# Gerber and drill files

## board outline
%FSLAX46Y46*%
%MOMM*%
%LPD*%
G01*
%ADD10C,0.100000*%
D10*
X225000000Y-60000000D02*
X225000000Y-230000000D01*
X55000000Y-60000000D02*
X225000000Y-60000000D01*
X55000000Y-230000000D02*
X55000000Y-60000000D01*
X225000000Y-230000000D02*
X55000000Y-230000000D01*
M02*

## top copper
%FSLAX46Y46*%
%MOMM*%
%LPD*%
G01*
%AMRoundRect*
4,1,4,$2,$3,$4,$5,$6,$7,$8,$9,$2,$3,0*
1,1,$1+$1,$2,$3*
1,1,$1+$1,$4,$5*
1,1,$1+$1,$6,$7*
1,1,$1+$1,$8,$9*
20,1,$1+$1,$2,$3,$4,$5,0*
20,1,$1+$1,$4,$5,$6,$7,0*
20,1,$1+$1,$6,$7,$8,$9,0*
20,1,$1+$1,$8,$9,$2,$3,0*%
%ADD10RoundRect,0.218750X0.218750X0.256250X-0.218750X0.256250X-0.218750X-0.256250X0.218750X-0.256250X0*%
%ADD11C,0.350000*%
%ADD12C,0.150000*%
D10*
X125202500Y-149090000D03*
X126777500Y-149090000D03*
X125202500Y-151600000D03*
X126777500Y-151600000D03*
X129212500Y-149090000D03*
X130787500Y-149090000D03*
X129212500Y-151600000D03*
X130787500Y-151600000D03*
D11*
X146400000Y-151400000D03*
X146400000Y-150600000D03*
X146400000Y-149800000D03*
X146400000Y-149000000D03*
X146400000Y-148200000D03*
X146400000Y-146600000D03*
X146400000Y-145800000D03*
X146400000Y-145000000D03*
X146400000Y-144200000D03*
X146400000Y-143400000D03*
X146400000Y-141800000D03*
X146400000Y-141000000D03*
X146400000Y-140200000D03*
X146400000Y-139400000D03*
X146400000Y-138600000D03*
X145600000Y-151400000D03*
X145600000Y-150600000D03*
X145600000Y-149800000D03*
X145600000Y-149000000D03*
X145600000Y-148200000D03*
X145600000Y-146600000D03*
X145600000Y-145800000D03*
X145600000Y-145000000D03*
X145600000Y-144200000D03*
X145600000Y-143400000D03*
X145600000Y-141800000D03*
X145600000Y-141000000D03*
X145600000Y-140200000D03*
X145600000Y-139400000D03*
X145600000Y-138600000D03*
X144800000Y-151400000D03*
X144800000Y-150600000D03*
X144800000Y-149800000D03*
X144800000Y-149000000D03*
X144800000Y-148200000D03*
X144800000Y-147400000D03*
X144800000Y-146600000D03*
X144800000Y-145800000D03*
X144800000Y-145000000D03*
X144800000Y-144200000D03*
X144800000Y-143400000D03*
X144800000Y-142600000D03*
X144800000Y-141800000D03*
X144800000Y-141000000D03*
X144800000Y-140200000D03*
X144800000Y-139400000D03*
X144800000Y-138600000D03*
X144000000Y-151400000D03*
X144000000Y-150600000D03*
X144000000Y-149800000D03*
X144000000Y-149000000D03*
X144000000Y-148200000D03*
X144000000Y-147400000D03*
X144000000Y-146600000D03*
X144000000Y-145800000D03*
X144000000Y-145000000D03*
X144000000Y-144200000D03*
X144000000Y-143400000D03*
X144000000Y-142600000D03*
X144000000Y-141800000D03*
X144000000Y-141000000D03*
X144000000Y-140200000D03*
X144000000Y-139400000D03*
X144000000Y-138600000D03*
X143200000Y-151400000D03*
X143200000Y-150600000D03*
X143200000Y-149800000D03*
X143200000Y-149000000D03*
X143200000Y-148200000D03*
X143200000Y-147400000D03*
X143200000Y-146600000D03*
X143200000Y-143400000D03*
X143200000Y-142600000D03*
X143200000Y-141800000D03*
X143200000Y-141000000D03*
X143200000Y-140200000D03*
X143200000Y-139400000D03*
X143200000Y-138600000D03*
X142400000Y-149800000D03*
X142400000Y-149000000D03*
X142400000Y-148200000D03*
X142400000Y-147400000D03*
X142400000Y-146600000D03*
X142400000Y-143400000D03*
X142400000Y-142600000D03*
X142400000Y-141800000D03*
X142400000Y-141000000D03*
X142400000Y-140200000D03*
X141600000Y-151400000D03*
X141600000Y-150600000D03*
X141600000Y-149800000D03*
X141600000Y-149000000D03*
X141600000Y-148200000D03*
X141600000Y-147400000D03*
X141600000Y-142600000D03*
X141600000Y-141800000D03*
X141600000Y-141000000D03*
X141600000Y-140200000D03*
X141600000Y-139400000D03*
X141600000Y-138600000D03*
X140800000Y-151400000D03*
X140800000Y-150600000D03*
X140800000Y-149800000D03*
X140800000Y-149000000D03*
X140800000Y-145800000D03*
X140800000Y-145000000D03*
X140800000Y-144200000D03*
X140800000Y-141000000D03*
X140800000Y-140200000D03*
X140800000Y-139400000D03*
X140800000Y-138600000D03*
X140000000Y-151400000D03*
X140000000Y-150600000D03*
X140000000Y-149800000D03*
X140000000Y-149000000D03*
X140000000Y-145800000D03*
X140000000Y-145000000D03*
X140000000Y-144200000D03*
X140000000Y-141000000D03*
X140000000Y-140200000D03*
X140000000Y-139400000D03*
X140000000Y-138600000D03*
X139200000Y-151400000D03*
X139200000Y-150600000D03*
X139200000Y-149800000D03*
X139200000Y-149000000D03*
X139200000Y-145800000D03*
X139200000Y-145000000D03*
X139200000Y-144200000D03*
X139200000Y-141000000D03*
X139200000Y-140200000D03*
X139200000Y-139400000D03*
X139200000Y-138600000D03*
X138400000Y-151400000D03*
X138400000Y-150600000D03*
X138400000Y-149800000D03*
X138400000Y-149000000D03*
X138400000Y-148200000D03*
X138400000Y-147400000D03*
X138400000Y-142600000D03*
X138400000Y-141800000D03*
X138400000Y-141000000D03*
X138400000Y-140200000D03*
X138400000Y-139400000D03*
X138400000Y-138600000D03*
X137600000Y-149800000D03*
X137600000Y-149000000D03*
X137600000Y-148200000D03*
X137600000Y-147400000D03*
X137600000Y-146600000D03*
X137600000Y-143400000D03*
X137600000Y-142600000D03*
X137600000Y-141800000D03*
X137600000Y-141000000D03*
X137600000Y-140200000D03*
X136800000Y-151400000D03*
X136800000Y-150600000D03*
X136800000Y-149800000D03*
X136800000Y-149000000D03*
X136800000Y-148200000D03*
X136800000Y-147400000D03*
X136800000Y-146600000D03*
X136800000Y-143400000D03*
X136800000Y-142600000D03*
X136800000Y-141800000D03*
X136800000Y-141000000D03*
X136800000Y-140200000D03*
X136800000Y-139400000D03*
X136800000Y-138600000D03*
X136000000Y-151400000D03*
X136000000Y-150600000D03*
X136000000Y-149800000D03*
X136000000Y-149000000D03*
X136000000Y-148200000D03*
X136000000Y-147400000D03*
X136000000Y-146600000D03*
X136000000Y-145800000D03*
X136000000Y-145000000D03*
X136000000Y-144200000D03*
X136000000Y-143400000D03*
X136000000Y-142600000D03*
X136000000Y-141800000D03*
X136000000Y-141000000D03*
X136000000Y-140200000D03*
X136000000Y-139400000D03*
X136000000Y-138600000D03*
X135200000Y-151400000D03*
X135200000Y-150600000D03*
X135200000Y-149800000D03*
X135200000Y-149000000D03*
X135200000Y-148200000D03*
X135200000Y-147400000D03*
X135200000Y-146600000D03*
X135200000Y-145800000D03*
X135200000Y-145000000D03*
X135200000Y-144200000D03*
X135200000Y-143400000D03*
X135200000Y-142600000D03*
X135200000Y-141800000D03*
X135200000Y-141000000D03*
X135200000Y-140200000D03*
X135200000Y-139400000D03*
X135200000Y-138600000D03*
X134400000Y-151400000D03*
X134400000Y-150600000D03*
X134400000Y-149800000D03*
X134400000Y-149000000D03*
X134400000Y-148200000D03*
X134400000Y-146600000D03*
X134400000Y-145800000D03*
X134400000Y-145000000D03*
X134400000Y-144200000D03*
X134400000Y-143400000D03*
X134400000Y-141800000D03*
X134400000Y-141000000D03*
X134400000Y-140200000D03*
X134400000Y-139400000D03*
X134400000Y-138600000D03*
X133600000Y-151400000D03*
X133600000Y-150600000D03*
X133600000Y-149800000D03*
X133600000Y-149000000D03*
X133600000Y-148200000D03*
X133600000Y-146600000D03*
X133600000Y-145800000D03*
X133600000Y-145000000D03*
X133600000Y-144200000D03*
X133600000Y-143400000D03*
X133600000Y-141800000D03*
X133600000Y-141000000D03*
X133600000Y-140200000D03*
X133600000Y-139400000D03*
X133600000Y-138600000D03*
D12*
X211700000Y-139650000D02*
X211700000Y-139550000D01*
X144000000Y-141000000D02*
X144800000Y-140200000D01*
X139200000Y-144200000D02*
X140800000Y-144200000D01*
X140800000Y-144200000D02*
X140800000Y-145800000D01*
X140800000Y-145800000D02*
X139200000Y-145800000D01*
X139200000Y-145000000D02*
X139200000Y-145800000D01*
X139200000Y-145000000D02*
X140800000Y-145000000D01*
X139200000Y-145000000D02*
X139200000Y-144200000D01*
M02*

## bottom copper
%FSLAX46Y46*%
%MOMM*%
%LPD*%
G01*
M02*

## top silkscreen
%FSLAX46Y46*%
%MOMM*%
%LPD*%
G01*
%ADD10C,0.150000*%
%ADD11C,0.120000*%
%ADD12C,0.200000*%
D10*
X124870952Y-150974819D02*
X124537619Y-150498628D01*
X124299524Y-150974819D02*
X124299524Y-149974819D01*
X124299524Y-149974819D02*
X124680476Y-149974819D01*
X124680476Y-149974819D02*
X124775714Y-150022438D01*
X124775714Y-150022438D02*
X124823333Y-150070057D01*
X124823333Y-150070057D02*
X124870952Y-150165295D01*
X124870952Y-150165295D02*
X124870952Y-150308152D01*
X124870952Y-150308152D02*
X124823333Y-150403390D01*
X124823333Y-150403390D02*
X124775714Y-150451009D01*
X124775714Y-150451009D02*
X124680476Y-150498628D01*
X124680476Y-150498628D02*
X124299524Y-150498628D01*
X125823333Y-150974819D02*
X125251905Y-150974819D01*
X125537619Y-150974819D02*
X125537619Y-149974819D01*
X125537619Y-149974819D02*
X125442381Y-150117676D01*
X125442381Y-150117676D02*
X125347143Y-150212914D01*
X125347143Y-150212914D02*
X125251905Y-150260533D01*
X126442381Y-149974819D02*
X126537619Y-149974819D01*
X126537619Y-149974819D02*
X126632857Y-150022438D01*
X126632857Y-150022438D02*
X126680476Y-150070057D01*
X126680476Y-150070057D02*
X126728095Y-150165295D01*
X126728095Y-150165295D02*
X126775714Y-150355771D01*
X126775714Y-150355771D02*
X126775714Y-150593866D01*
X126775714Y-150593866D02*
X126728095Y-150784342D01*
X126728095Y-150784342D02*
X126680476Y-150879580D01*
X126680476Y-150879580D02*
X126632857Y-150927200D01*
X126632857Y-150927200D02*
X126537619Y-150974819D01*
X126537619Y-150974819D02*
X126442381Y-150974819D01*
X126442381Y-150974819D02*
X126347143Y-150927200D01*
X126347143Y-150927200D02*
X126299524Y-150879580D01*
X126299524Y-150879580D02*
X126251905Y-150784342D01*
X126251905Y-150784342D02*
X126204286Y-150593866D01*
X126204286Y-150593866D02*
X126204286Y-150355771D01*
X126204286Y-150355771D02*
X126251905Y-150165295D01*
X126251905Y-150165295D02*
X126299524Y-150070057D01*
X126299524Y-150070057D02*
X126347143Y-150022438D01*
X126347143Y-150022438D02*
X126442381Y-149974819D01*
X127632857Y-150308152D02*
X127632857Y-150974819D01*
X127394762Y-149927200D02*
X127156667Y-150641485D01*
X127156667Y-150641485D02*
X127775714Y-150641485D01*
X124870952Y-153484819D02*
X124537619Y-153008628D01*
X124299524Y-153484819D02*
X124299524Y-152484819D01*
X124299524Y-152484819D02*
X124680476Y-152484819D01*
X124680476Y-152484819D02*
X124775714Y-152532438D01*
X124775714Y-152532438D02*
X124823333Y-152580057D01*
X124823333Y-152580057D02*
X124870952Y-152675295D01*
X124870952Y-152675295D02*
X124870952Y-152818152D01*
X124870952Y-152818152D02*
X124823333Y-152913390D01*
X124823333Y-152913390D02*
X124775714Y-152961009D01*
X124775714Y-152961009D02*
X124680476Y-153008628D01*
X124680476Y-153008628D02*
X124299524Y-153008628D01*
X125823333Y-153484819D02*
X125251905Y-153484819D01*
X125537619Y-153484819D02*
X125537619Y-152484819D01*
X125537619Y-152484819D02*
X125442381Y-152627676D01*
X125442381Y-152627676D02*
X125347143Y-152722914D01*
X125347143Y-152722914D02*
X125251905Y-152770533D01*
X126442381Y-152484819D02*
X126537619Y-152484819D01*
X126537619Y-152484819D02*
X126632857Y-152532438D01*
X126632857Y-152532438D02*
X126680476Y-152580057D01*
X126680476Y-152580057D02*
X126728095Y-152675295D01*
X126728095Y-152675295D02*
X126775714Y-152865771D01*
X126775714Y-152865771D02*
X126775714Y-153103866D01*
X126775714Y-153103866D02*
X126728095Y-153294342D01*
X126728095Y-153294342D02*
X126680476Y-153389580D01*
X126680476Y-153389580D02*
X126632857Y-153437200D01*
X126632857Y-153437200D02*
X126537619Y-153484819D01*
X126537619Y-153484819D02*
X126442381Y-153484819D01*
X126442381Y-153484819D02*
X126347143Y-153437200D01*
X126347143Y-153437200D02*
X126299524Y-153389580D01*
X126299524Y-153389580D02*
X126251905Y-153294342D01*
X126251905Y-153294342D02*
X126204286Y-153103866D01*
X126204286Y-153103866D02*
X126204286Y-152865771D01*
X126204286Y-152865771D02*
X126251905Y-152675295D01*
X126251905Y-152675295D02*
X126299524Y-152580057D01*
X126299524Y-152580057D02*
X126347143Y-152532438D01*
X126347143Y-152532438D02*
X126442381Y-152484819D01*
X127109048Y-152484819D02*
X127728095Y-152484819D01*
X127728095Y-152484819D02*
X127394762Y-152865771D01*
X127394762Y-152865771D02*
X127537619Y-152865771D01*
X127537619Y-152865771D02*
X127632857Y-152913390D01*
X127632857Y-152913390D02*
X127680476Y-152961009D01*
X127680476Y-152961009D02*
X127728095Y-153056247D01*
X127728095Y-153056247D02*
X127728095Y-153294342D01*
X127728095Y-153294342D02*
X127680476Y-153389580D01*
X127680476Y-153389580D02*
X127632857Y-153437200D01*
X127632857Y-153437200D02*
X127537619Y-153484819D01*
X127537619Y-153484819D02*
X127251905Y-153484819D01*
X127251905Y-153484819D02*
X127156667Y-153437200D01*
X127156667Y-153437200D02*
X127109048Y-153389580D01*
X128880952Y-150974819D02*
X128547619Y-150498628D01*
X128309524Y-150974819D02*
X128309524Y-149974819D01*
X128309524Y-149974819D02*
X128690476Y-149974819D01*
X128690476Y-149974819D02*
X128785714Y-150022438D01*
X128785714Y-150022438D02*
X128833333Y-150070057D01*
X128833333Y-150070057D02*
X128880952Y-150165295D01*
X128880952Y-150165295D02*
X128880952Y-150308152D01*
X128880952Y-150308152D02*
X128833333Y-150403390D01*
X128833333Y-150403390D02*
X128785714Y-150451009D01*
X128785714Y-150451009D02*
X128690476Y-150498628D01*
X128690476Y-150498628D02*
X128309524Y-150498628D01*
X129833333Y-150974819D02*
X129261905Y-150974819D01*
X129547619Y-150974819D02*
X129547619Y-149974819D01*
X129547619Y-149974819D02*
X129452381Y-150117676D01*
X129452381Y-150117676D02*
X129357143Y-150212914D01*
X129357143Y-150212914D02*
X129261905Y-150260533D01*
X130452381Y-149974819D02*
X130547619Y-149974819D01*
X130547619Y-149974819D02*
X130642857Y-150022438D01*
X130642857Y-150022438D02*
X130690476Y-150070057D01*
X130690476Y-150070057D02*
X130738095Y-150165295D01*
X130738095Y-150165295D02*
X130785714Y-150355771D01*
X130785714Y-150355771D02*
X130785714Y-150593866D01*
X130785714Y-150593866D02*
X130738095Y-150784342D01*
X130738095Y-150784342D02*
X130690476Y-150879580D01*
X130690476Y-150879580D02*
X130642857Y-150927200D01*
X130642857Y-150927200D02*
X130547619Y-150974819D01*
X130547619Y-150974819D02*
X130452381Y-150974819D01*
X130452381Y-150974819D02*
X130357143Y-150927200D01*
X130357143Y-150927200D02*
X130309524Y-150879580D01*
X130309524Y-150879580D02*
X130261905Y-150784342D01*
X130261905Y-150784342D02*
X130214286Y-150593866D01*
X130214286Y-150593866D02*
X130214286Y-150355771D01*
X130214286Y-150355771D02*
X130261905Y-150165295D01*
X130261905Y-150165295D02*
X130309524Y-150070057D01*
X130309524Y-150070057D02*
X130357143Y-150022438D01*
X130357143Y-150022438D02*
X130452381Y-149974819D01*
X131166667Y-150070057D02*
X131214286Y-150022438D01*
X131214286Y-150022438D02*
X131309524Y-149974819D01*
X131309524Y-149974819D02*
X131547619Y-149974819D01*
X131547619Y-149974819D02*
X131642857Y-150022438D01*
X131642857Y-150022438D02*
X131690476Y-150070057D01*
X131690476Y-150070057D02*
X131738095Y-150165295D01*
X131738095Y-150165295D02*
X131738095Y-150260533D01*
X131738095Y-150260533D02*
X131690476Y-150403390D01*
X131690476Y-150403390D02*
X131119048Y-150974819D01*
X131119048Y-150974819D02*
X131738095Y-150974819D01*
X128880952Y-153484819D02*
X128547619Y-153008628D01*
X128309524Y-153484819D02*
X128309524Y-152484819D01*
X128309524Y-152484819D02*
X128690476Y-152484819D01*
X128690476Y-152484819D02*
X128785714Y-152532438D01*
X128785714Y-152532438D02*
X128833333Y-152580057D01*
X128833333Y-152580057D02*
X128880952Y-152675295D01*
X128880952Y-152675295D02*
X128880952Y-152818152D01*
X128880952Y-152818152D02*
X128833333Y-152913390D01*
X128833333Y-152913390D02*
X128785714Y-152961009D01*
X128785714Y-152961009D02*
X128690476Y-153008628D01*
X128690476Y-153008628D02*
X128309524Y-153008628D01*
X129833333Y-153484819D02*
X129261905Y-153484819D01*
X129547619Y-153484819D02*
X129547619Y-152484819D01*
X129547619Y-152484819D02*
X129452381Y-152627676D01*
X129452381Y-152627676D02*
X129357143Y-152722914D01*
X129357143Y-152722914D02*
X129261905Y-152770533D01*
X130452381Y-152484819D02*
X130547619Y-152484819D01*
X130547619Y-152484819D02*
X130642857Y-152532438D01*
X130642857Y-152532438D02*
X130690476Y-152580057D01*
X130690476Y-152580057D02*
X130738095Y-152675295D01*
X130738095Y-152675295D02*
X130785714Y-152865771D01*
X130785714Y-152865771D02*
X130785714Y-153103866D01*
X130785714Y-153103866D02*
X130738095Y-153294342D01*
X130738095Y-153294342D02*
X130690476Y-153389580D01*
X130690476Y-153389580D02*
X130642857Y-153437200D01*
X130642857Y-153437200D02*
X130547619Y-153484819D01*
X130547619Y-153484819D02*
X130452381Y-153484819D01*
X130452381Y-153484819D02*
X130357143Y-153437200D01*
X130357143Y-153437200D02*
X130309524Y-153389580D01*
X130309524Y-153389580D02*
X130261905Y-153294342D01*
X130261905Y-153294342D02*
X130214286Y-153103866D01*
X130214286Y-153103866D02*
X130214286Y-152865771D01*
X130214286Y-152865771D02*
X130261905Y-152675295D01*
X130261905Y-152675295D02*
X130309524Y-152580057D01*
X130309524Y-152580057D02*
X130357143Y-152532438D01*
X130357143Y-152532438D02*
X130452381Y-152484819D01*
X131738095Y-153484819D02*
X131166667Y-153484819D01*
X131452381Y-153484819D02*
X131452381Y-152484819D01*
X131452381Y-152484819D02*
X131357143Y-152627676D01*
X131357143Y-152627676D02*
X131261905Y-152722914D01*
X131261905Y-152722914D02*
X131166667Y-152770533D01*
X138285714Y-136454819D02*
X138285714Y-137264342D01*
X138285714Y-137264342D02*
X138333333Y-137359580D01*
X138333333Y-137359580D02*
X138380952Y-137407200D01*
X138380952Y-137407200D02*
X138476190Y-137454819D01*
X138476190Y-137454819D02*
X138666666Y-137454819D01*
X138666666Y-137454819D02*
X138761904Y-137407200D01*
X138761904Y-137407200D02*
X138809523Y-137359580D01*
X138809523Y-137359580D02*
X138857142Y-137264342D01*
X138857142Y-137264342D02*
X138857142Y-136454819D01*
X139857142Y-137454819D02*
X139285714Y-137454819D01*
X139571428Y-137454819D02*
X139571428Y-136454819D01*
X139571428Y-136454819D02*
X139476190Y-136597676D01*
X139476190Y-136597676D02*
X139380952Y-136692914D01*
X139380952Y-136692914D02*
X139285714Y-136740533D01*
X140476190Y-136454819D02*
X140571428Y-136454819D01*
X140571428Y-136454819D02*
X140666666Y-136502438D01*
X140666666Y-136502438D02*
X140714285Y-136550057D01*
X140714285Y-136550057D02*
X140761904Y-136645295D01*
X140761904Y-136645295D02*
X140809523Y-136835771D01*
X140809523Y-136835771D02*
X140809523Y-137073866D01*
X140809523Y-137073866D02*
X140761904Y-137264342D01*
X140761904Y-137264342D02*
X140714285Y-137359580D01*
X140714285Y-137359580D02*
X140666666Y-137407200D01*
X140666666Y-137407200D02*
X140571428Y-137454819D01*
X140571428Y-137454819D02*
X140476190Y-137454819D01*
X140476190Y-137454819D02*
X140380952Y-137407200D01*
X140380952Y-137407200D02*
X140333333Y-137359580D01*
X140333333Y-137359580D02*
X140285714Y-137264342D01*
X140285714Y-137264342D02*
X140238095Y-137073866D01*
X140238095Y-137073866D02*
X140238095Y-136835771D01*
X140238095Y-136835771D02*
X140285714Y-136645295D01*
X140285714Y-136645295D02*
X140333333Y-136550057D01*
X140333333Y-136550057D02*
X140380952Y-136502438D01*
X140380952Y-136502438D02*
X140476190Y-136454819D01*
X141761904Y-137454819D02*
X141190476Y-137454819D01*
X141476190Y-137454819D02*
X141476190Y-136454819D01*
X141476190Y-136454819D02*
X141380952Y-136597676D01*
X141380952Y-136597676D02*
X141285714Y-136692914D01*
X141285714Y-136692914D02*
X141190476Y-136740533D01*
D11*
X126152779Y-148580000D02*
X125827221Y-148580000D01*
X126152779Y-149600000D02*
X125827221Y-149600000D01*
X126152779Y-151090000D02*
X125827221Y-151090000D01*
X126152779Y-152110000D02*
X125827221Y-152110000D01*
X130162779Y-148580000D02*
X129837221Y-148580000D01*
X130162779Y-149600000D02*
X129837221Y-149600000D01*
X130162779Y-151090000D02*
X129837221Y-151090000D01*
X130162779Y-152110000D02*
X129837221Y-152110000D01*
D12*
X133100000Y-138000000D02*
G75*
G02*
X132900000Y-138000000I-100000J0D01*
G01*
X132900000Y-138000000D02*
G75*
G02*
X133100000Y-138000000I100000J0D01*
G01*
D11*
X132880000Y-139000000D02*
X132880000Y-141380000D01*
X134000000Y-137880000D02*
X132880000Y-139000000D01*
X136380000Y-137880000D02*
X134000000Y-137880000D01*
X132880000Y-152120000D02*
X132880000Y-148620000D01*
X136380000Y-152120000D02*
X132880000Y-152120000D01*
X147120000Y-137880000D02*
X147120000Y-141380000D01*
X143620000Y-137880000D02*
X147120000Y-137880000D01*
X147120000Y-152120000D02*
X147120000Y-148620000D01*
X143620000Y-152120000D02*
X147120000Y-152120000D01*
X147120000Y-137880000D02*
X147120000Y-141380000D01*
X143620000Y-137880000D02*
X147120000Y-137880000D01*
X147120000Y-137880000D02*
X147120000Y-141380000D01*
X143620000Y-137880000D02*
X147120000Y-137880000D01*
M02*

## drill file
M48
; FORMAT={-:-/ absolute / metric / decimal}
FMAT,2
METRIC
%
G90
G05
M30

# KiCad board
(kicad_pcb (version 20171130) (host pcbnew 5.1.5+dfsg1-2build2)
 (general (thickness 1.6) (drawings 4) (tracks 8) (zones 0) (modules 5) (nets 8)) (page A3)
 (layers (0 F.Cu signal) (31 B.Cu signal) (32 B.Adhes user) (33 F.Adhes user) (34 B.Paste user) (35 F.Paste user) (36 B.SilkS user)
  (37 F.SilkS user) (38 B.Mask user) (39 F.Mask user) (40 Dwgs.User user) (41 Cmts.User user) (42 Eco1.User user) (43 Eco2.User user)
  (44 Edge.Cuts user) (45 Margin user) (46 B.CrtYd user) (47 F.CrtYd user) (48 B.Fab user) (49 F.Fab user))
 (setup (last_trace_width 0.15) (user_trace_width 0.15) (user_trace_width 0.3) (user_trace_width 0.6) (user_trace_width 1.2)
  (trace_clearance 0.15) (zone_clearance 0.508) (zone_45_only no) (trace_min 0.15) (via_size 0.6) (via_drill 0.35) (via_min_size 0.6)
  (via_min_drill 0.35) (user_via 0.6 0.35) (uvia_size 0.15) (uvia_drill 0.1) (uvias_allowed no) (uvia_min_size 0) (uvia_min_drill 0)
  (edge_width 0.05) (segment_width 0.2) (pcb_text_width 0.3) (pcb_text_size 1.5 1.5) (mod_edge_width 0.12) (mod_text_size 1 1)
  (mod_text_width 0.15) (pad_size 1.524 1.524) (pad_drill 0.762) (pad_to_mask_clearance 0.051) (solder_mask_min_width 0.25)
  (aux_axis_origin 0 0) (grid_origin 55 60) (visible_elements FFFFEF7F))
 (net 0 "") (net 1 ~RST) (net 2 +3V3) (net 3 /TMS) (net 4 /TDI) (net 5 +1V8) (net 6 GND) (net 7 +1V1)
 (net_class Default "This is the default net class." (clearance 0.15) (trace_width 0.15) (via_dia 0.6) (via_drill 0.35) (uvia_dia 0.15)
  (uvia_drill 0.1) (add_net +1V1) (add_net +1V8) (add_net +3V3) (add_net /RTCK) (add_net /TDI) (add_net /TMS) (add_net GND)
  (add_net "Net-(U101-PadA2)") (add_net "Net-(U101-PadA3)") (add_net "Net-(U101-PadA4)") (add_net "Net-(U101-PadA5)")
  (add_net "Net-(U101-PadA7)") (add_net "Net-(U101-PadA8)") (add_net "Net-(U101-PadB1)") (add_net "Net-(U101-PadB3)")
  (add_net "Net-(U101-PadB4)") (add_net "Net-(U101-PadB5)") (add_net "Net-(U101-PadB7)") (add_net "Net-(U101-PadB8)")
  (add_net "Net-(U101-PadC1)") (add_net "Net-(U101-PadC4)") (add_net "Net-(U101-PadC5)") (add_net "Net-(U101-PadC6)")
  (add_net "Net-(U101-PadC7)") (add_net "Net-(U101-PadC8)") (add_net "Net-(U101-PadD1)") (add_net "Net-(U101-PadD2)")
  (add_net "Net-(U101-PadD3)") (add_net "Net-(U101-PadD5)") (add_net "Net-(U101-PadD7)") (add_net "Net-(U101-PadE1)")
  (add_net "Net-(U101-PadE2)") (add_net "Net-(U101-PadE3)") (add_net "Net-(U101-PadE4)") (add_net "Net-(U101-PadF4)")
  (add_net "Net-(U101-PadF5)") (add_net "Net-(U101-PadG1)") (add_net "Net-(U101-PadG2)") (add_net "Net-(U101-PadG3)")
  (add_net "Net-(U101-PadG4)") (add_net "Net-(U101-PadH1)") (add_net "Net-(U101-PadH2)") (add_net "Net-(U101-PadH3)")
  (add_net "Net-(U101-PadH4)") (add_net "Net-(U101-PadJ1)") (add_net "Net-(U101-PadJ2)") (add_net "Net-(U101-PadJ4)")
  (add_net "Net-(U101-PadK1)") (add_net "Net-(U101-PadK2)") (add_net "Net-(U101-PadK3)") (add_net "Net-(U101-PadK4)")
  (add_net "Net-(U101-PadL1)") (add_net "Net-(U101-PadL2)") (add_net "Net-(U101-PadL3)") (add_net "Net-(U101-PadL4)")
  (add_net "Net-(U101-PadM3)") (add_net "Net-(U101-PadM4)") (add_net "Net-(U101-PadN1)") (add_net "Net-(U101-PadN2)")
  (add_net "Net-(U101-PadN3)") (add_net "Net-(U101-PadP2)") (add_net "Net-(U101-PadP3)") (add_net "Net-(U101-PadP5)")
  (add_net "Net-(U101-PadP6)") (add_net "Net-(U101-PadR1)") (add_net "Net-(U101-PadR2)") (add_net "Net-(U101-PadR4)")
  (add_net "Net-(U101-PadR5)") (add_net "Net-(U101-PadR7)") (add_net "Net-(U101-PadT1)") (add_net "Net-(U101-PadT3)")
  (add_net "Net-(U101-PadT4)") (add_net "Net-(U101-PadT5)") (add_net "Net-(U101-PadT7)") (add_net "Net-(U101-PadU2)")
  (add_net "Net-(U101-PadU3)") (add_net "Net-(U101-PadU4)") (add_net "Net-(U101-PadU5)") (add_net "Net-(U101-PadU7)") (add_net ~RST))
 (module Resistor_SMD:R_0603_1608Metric (layer F.Cu) (at 125.99 149.09 180)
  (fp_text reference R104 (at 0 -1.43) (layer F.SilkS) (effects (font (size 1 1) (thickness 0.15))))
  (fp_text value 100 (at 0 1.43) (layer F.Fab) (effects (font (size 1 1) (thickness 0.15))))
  (fp_line (start -0.162779 0.51) (end 0.162779 0.51) (layer F.SilkS) (width 0.12))
  (fp_line (start -0.162779 -0.51) (end 0.162779 -0.51) (layer F.SilkS) (width 0.12))
  (pad 2 smd roundrect (at 0.7875 0 180) (size 0.875 0.95) (layers F.Cu F.Paste F.Mask) (roundrect_rratio 0.25))
  (pad 1 smd roundrect (at -0.7875 0 180) (size 0.875 0.95) (layers F.Cu F.Paste F.Mask) (roundrect_rratio 0.25) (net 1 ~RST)))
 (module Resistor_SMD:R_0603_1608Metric (layer F.Cu) (at 125.99 151.6 180)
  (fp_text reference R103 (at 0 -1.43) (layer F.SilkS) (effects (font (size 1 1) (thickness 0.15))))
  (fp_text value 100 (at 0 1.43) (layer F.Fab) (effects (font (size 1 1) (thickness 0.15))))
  (fp_line (start -0.162779 0.51) (end 0.162779 0.51) (layer F.SilkS) (width 0.12))
  (fp_line (start -0.162779 -0.51) (end 0.162779 -0.51) (layer F.SilkS) (width 0.12))
  (pad 2 smd roundrect (at 0.7875 0 180) (size 0.875 0.95) (layers F.Cu F.Paste F.Mask) (roundrect_rratio 0.25) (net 1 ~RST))
  (pad 1 smd roundrect (at -0.7875 0 180) (size 0.875 0.95) (layers F.Cu F.Paste F.Mask) (roundrect_rratio 0.25) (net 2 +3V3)))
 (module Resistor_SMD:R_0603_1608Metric (layer F.Cu) (at 130 149.09 180)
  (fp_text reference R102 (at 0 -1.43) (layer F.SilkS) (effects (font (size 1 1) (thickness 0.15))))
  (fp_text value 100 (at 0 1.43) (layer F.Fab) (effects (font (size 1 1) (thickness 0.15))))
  (fp_line (start -0.162779 0.51) (end 0.162779 0.51) (layer F.SilkS) (width 0.12))
  (fp_line (start -0.162779 -0.51) (end 0.162779 -0.51) (layer F.SilkS) (width 0.12))
  (pad 2 smd roundrect (at 0.7875 0 180) (size 0.875 0.95) (layers F.Cu F.Paste F.Mask) (roundrect_rratio 0.25) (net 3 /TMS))
  (pad 1 smd roundrect (at -0.7875 0 180) (size 0.875 0.95) (layers F.Cu F.Paste F.Mask) (roundrect_rratio 0.25) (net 2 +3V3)))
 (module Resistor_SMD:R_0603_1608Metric (layer F.Cu) (at 130 151.6 180)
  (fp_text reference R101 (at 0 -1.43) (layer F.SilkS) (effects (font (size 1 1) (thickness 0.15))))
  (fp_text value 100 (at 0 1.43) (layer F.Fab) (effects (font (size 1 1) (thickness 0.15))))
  (fp_line (start -0.162779 0.51) (end 0.162779 0.51) (layer F.SilkS) (width 0.12))
  (fp_line (start -0.162779 -0.51) (end 0.162779 -0.51) (layer F.SilkS) (width 0.12))
  (pad 2 smd roundrect (at 0.7875 0 180) (size 0.875 0.95) (layers F.Cu F.Paste F.Mask) (roundrect_rratio 0.25) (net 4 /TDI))
  (pad 1 smd roundrect (at -0.7875 0 180) (size 0.875 0.95) (layers F.Cu F.Paste F.Mask) (roundrect_rratio 0.25) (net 2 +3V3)))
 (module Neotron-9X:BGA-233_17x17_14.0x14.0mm (layer F.Cu) (at 140 145)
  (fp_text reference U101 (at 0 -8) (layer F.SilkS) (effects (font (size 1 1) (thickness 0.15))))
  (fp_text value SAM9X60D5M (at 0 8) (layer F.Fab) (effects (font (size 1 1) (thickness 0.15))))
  (fp_circle (center -7 -7) (end -7 -6.9) (layer F.SilkS) (width 0.2))
  (fp_line (start -7.12 -6) (end -7.12 -3.62) (layer F.SilkS) (width 0.12))
  (fp_line (start -6 -7.12) (end -7.12 -6) (layer F.SilkS) (width 0.12))
  (fp_line (start -3.62 -7.12) (end -6 -7.12) (layer F.SilkS) (width 0.12))
  (fp_line (start -7.12 7.12) (end -7.12 3.62) (layer F.SilkS) (width 0.12))
  (fp_line (start -3.62 7.12) (end -7.12 7.12) (layer F.SilkS) (width 0.12))
  (fp_line (start 7.12 -7.12) (end 7.12 -3.62) (layer F.SilkS) (width 0.12))
  (fp_line (start 3.62 -7.12) (end 7.12 -7.12) (layer F.SilkS) (width 0.12))
  (fp_line (start 7.12 7.12) (end 7.12 3.62) (layer F.SilkS) (width 0.12))
  (fp_line (start 3.62 7.12) (end 7.12 7.12) (layer F.SilkS) (width 0.12))
  (fp_line (start 7.12 -7.12) (end 7.12 -3.62) (layer F.SilkS) (width 0.12))
  (fp_line (start 3.62 -7.12) (end 7.12 -7.12) (layer F.SilkS) (width 0.12))
  (fp_line (start 7.12 -7.12) (end 7.12 -3.62) (layer F.SilkS) (width 0.12))
  (fp_line (start 3.62 -7.12) (end 7.12 -7.12) (layer F.SilkS) (width 0.12))
  (pad U17 smd circle (at 6.4 6.4) (size 0.35 0.35) (layers F.Cu F.Paste F.Mask))
  (pad T17 smd circle (at 6.4 5.6) (size 0.35 0.35) (layers F.Cu F.Paste F.Mask))
  (pad R17 smd circle (at 6.4 4.8) (size 0.35 0.35) (layers F.Cu F.Paste F.Mask))
  (pad P17 smd circle (at 6.4 4) (size 0.35 0.35) (layers F.Cu F.Paste F.Mask))
  (pad N17 smd circle (at 6.4 3.2) (size 0.35 0.35) (layers F.Cu F.Paste F.Mask))
  (pad L17 smd circle (at 6.4 1.6) (size 0.35 0.35) (layers F.Cu F.Paste F.Mask))
  (pad K17 smd circle (at 6.4 0.8) (size 0.35 0.35) (layers F.Cu F.Paste F.Mask))
  (pad J17 smd circle (at 6.4 0) (size 0.35 0.35) (layers F.Cu F.Paste F.Mask))
  (pad H17 smd circle (at 6.4 -0.8) (size 0.35 0.35) (layers F.Cu F.Paste F.Mask))
  (pad G17 smd circle (at 6.4 -1.6) (size 0.35 0.35) (layers F.Cu F.Paste F.Mask))
  (pad E17 smd circle (at 6.4 -3.2) (size 0.35 0.35) (layers F.Cu F.Paste F.Mask))
  (pad D17 smd circle (at 6.4 -4) (size 0.35 0.35) (layers F.Cu F.Paste F.Mask))
  (pad C17 smd circle (at 6.4 -4.8) (size 0.35 0.35) (layers F.Cu F.Paste F.Mask))
  (pad B17 smd circle (at 6.4 -5.6) (size 0.35 0.35) (layers F.Cu F.Paste F.Mask) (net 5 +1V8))
  (pad A17 smd circle (at 6.4 -6.4) (size 0.35 0.35) (layers F.Cu F.Paste F.Mask) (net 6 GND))
  (pad U16 smd circle (at 5.6 6.4) (size 0.35 0.35) (layers F.Cu F.Paste F.Mask))
  (pad T16 smd circle (at 5.6 5.6) (size 0.35 0.35) (layers F.Cu F.Paste F.Mask) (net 6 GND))
  (pad R16 smd circle (at 5.6 4.8) (size 0.35 0.35) (layers F.Cu F.Paste F.Mask) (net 6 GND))
  (pad P16 smd circle (at 5.6 4) (size 0.35 0.35) (layers F.Cu F.Paste F.Mask))
  (pad N16 smd circle (at 5.6 3.2) (size 0.35 0.35) (layers F.Cu F.Paste F.Mask) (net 3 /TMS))
  (pad L16 smd circle (at 5.6 1.6) (size 0.35 0.35) (layers F.Cu F.Paste F.Mask))
  (pad K16 smd circle (at 5.6 0.8) (size 0.35 0.35) (layers F.Cu F.Paste F.Mask))
  (pad J16 smd circle (at 5.6 0) (size 0.35 0.35) (layers F.Cu F.Paste F.Mask))
  (pad H16 smd circle (at 5.6 -0.8) (size 0.35 0.35) (layers F.Cu F.Paste F.Mask))
  (pad G16 smd circle (at 5.6 -1.6) (size 0.35 0.35) (layers F.Cu F.Paste F.Mask))
  (pad E16 smd circle (at 5.6 -3.2) (size 0.35 0.35) (layers F.Cu F.Paste F.Mask))
  (pad D16 smd circle (at 5.6 -4) (size 0.35 0.35) (layers F.Cu F.Paste F.Mask))
  (pad C16 smd circle (at 5.6 -4.8) (size 0.35 0.35) (layers F.Cu F.Paste F.Mask) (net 5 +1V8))
  (pad B16 smd circle (at 5.6 -5.6) (size 0.35 0.35) (layers F.Cu F.Paste F.Mask) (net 6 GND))
  (pad A16 smd circle (at 5.6 -6.4) (size 0.35 0.35) (layers F.Cu F.Paste F.Mask) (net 5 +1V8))
  (pad U15 smd circle (at 4.8 6.4) (size 0.35 0.35) (layers F.Cu F.Paste F.Mask) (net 6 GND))
  (pad T15 smd circle (at 4.8 5.6) (size 0.35 0.35) (layers F.Cu F.Paste F.Mask))
  (pad R15 smd circle (at 4.8 4.8) (size 0.35 0.35) (layers F.Cu F.Paste F.Mask) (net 6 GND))
  (pad P15 smd circle (at 4.8 4) (size 0.35 0.35) (layers F.Cu F.Paste F.Mask))
  (pad N15 smd circle (at 4.8 3.2) (size 0.35 0.35) (layers F.Cu F.Paste F.Mask))
  (pad M15 smd circle (at 4.8 2.4) (size 0.35 0.35) (layers F.Cu F.Paste F.Mask))
  (pad L15 smd circle (at 4.8 1.6) (size 0.35 0.35) (layers F.Cu F.Paste F.Mask) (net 4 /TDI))
  (pad K15 smd circle (at 4.8 0.8) (size 0.35 0.35) (layers F.Cu F.Paste F.Mask))
  (pad J15 smd circle (at 4.8 0) (size 0.35 0.35) (layers F.Cu F.Paste F.Mask) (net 6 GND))
  (pad H15 smd circle (at 4.8 -0.8) (size 0.35 0.35) (layers F.Cu F.Paste F.Mask))
  (pad G15 smd circle (at 4.8 -1.6) (size 0.35 0.35) (layers F.Cu F.Paste F.Mask))
  (pad F15 smd circle (at 4.8 -2.4) (size 0.35 0.35) (layers F.Cu F.Paste F.Mask) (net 6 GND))
  (pad E15 smd circle (at 4.8 -3.2) (size 0.35 0.35) (layers F.Cu F.Paste F.Mask))
  (pad D15 smd circle (at 4.8 -4) (size 0.35 0.35) (layers F.Cu F.Paste F.Mask) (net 5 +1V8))
  (pad C15 smd circle (at 4.8 -4.8) (size 0.35 0.35) (layers F.Cu F.Paste F.Mask) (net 6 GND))
  (pad B15 smd circle (at 4.8 -5.6) (size 0.35 0.35) (layers F.Cu F.Paste F.Mask) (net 5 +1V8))
  (pad A15 smd circle (at 4.8 -6.4) (size 0.35 0.35) (layers F.Cu F.Paste F.Mask) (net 6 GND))
  (pad U14 smd circle (at 4 6.4) (size 0.35 0.35) (layers F.Cu F.Paste F.Mask))
  (pad T14 smd circle (at 4 5.6) (size 0.35 0.35) (layers F.Cu F.Paste F.Mask))
  (pad R14 smd circle (at 4 4.8) (size 0.35 0.35) (layers F.Cu F.Paste F.Mask))
  (pad P14 smd circle (at 4 4) (size 0.35 0.35) (layers F.Cu F.Paste F.Mask) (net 6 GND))
  (pad N14 smd circle (at 4 3.2) (size 0.35 0.35) (layers F.Cu F.Paste F.Mask))
  (pad M14 smd circle (at 4 2.4) (size 0.35 0.35) (layers F.Cu F.Paste F.Mask) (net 6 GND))
  (pad L14 smd circle (at 4 1.6) (size 0.35 0.35) (layers F.Cu F.Paste F.Mask) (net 6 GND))
  (pad K14 smd circle (at 4 0.8) (size 0.35 0.35) (layers F.Cu F.Paste F.Mask))
  (pad J14 smd circle (at 4 0) (size 0.35 0.35) (layers F.Cu F.Paste F.Mask))
  (pad H14 smd circle (at 4 -0.8) (size 0.35 0.35) (layers F.Cu F.Paste F.Mask))
  (pad G14 smd circle (at 4 -1.6) (size 0.35 0.35) (layers F.Cu F.Paste F.Mask))
  (pad F14 smd circle (at 4 -2.4) (size 0.35 0.35) (layers F.Cu F.Paste F.Mask))
  (pad E14 smd circle (at 4 -3.2) (size 0.35 0.35) (layers F.Cu F.Paste F.Mask))
  (pad D14 smd circle (at 4 -4) (size 0.35 0.35) (layers F.Cu F.Paste F.Mask) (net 6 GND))
  (pad C14 smd circle (at 4 -4.8) (size 0.35 0.35) (layers F.Cu F.Paste F.Mask) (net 5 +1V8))
  (pad B14 smd circle (at 4 -5.6) (size 0.35 0.35) (layers F.Cu F.Paste F.Mask) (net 6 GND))
  (pad A14 smd circle (at 4 -6.4) (size 0.35 0.35) (layers F.Cu F.Paste F.Mask))
  (pad U13 smd circle (at 3.2 6.4) (size 0.35 0.35) (layers F.Cu F.Paste F.Mask))
  (pad T13 smd circle (at 3.2 5.6) (size 0.35 0.35) (layers F.Cu F.Paste F.Mask))
  (pad R13 smd circle (at 3.2 4.8) (size 0.35 0.35) (layers F.Cu F.Paste F.Mask))
  (pad P13 smd circle (at 3.2 4) (size 0.35 0.35) (layers F.Cu F.Paste F.Mask))
  (pad N13 smd circle (at 3.2 3.2) (size 0.35 0.35) (layers F.Cu F.Paste F.Mask) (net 6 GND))
  (pad M13 smd circle (at 3.2 2.4) (size 0.35 0.35) (layers F.Cu F.Paste F.Mask) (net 6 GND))
  (pad L13 smd circle (at 3.2 1.6) (size 0.35 0.35) (layers F.Cu F.Paste F.Mask) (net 6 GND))
  (pad G13 smd circle (at 3.2 -1.6) (size 0.35 0.35) (layers F.Cu F.Paste F.Mask) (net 5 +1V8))
  (pad F13 smd circle (at 3.2 -2.4) (size 0.35 0.35) (layers F.Cu F.Paste F.Mask) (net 5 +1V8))
  (pad E13 smd circle (at 3.2 -3.2) (size 0.35 0.35) (layers F.Cu F.Paste F.Mask) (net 6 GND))
  (pad D13 smd circle (at 3.2 -4) (size 0.35 0.35) (layers F.Cu F.Paste F.Mask) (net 5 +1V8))
  (pad C13 smd circle (at 3.2 -4.8) (size 0.35 0.35) (layers F.Cu F.Paste F.Mask) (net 6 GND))
  (pad B13 smd circle (at 3.2 -5.6) (size 0.35 0.35) (layers F.Cu F.Paste F.Mask) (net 6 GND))
  (pad A13 smd circle (at 3.2 -6.4) (size 0.35 0.35) (layers F.Cu F.Paste F.Mask) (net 6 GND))
  (pad R12 smd circle (at 2.4 4.8) (size 0.35 0.35) (layers F.Cu F.Paste F.Mask))
  (pad P12 smd circle (at 2.4 4) (size 0.35 0.35) (layers F.Cu F.Paste F.Mask))
  (pad N12 smd circle (at 2.4 3.2) (size 0.35 0.35) (layers F.Cu F.Paste F.Mask) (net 6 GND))
  (pad M12 smd circle (at 2.4 2.4) (size 0.35 0.35) (layers F.Cu F.Paste F.Mask) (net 6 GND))
  (pad L12 smd circle (at 2.4 1.6) (size 0.35 0.35) (layers F.Cu F.Paste F.Mask) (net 6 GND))
  (pad G12 smd circle (at 2.4 -1.6) (size 0.35 0.35) (layers F.Cu F.Paste F.Mask) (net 6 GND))
  (pad F12 smd circle (at 2.4 -2.4) (size 0.35 0.35) (layers F.Cu F.Paste F.Mask) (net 6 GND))
  (pad E12 smd circle (at 2.4 -3.2) (size 0.35 0.35) (layers F.Cu F.Paste F.Mask) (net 5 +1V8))
  (pad D12 smd circle (at 2.4 -4) (size 0.35 0.35) (layers F.Cu F.Paste F.Mask))
  (pad C12 smd circle (at 2.4 -4.8) (size 0.35 0.35) (layers F.Cu F.Paste F.Mask) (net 6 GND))
  (pad U11 smd circle (at 1.6 6.4) (size 0.35 0.35) (layers F.Cu F.Paste F.Mask))
  (pad T11 smd circle (at 1.6 5.6) (size 0.35 0.35) (layers F.Cu F.Paste F.Mask))
  (pad R11 smd circle (at 1.6 4.8) (size 0.35 0.35) (layers F.Cu F.Paste F.Mask) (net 6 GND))
  (pad P11 smd circle (at 1.6 4) (size 0.35 0.35) (layers F.Cu F.Paste F.Mask))
  (pad N11 smd circle (at 1.6 3.2) (size 0.35 0.35) (layers F.Cu F.Paste F.Mask))
  (pad M11 smd circle (at 1.6 2.4) (size 0.35 0.35) (layers F.Cu F.Paste F.Mask) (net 6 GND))
  (pad F11 smd circle (at 1.6 -2.4) (size 0.35 0.35) (layers F.Cu F.Paste F.Mask) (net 6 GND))
  (pad E11 smd circle (at 1.6 -3.2) (size 0.35 0.35) (layers F.Cu F.Paste F.Mask) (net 5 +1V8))
  (pad D11 smd circle (at 1.6 -4) (size 0.35 0.35) (layers F.Cu F.Paste F.Mask))
  (pad C11 smd circle (at 1.6 -4.8) (size 0.35 0.35) (layers F.Cu F.Paste F.Mask))
  (pad B11 smd circle (at 1.6 -5.6) (size 0.35 0.35) (layers F.Cu F.Paste F.Mask))
  (pad A11 smd circle (at 1.6 -6.4) (size 0.35 0.35) (layers F.Cu F.Paste F.Mask))
  (pad U10 smd circle (at 0.8 6.4) (size 0.35 0.35) (layers F.Cu F.Paste F.Mask))
  (pad T10 smd circle (at 0.8 5.6) (size 0.35 0.35) (layers F.Cu F.Paste F.Mask))
  (pad R10 smd circle (at 0.8 4.8) (size 0.35 0.35) (layers F.Cu F.Paste F.Mask))
  (pad P10 smd circle (at 0.8 4) (size 0.35 0.35) (layers F.Cu F.Paste F.Mask) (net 6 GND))
  (pad K10 smd circle (at 0.8 0.8) (size 0.35 0.35) (layers F.Cu F.Paste F.Mask) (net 6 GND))
  (pad J10 smd circle (at 0.8 0) (size 0.35 0.35) (layers F.Cu F.Paste F.Mask) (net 6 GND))
  (pad H10 smd circle (at 0.8 -0.8) (size 0.35 0.35) (layers F.Cu F.Paste F.Mask) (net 6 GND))
  (pad D10 smd circle (at 0.8 -4) (size 0.35 0.35) (layers F.Cu F.Paste F.Mask))
  (pad C10 smd circle (at 0.8 -4.8) (size 0.35 0.35) (layers F.Cu F.Paste F.Mask))
  (pad B10 smd circle (at 0.8 -5.6) (size 0.35 0.35) (layers F.Cu F.Paste F.Mask))
  (pad A10 smd circle (at 0.8 -6.4) (size 0.35 0.35) (layers F.Cu F.Paste F.Mask))
  (pad U9 smd circle (at 0 6.4) (size 0.35 0.35) (layers F.Cu F.Paste F.Mask))
  (pad T9 smd circle (at 0 5.6) (size 0.35 0.35) (layers F.Cu F.Paste F.Mask))
  (pad R9 smd circle (at 0 4.8) (size 0.35 0.35) (layers F.Cu F.Paste F.Mask) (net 6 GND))
  (pad P9 smd circle (at 0 4) (size 0.35 0.35) (layers F.Cu F.Paste F.Mask))
  (pad K9 smd circle (at 0 0.8) (size 0.35 0.35) (layers F.Cu F.Paste F.Mask) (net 6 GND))
  (pad J9 smd circle (at 0 0) (size 0.35 0.35) (layers F.Cu F.Paste F.Mask) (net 6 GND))
  (pad H9 smd circle (at 0 -0.8) (size 0.35 0.35) (layers F.Cu F.Paste F.Mask) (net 6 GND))
  (pad D9 smd circle (at 0 -4) (size 0.35 0.35) (layers F.Cu F.Paste F.Mask))
  (pad C9 smd circle (at 0 -4.8) (size 0.35 0.35) (layers F.Cu F.Paste F.Mask) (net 6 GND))
  (pad B9 smd circle (at 0 -5.6) (size 0.35 0.35) (layers F.Cu F.Paste F.Mask))
  (pad A9 smd circle (at 0 -6.4) (size 0.35 0.35) (layers F.Cu F.Paste F.Mask))
  (pad U8 smd circle (at -0.8 6.4) (size 0.35 0.35) (layers F.Cu F.Paste F.Mask))
  (pad T8 smd circle (at -0.8 5.6) (size 0.35 0.35) (layers F.Cu F.Paste F.Mask))
  (pad R8 smd circle (at -0.8 4.8) (size 0.35 0.35) (layers F.Cu F.Paste F.Mask))
  (pad P8 smd circle (at -0.8 4) (size 0.35 0.35) (layers F.Cu F.Paste F.Mask))
  (pad K8 smd circle (at -0.8 0.8) (size 0.35 0.35) (layers F.Cu F.Paste F.Mask) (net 6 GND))
  (pad J8 smd circle (at -0.8 0) (size 0.35 0.35) (layers F.Cu F.Paste F.Mask) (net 6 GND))
  (pad H8 smd circle (at -0.8 -0.8) (size 0.35 0.35) (layers F.Cu F.Paste F.Mask) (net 6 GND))
  (pad D8 smd circle (at -0.8 -4) (size 0.35 0.35) (layers F.Cu F.Paste F.Mask) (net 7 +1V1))
  (pad C8 smd circle (at -0.8 -4.8) (size 0.35 0.35) (layers F.Cu F.Paste F.Mask))
  (pad B8 smd circle (at -0.8 -5.6) (size 0.35 0.35) (layers F.Cu F.Paste F.Mask))
  (pad A8 smd circle (at -0.8 -6.4) (size 0.35 0.35) (layers F.Cu F.Paste F.Mask))
  (pad U7 smd circle (at -1.6 6.4) (size 0.35 0.35) (layers F.Cu F.Paste F.Mask))
  (pad T7 smd circle (at -1.6 5.6) (size 0.35 0.35) (layers F.Cu F.Paste F.Mask))
  (pad R7 smd circle (at -1.6 4.8) (size 0.35 0.35) (layers F.Cu F.Paste F.Mask))
  (pad P7 smd circle (at -1.6 4) (size 0.35 0.35) (layers F.Cu F.Paste F.Mask) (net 6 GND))
  (pad N7 smd circle (at -1.6 3.2) (size 0.35 0.35) (layers F.Cu F.Paste F.Mask) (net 6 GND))
  (pad M7 smd circle (at -1.6 2.4) (size 0.35 0.35) (layers F.Cu F.Paste F.Mask) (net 7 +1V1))
  (pad F7 smd circle (at -1.6 -2.4) (size 0.35 0.35) (layers F.Cu F.Paste F.Mask) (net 6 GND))
  (pad E7 smd circle (at -1.6 -3.2) (size 0.35 0.35) (layers F.Cu F.Paste F.Mask) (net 6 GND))
  (pad D7 smd circle (at -1.6 -4) (size 0.35 0.35) (layers F.Cu F.Paste F.Mask))
  (pad C7 smd circle (at -1.6 -4.8) (size 0.35 0.35) (layers F.Cu F.Paste F.Mask))
  (pad B7 smd circle (at -1.6 -5.6) (size 0.35 0.35) (layers F.Cu F.Paste F.Mask))
  (pad A7 smd circle (at -1.6 -6.4) (size 0.35 0.35) (layers F.Cu F.Paste F.Mask))
  (pad R6 smd circle (at -2.4 4.8) (size 0.35 0.35) (layers F.Cu F.Paste F.Mask) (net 7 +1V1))
  (pad P6 smd circle (at -2.4 4) (size 0.35 0.35) (layers F.Cu F.Paste F.Mask))
  (pad N6 smd circle (at -2.4 3.2) (size 0.35 0.35) (layers F.Cu F.Paste F.Mask) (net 6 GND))
  (pad M6 smd circle (at -2.4 2.4) (size 0.35 0.35) (layers F.Cu F.Paste F.Mask) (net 6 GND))
  (pad L6 smd circle (at -2.4 1.6) (size 0.35 0.35) (layers F.Cu F.Paste F.Mask) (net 7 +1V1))
  (pad G6 smd circle (at -2.4 -1.6) (size 0.35 0.35) (layers F.Cu F.Paste F.Mask) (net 6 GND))
  (pad F6 smd circle (at -2.4 -2.4) (size 0.35 0.35) (layers F.Cu F.Paste F.Mask) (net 6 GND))
  (pad E6 smd circle (at -2.4 -3.2) (size 0.35 0.35) (layers F.Cu F.Paste F.Mask) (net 6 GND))
  (pad D6 smd circle (at -2.4 -4) (size 0.35 0.35) (layers F.Cu F.Paste F.Mask) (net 7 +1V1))
  (pad C6 smd circle (at -2.4 -4.8) (size 0.35 0.35) (layers F.Cu F.Paste F.Mask))
  (pad U5 smd circle (at -3.2 6.4) (size 0.35 0.35) (layers F.Cu F.Paste F.Mask))
  (pad T5 smd circle (at -3.2 5.6) (size 0.35 0.35) (layers F.Cu F.Paste F.Mask))
  (pad R5 smd circle (at -3.2 4.8) (size 0.35 0.35) (layers F.Cu F.Paste F.Mask))
  (pad P5 smd circle (at -3.2 4) (size 0.35 0.35) (layers F.Cu F.Paste F.Mask))
  (pad N5 smd circle (at -3.2 3.2) (size 0.35 0.35) (layers F.Cu F.Paste F.Mask) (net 6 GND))
  (pad M5 smd circle (at -3.2 2.4) (size 0.35 0.35) (layers F.Cu F.Paste F.Mask) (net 6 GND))
  (pad L5 smd circle (at -3.2 1.6) (size 0.35 0.35) (layers F.Cu F.Paste F.Mask) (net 6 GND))
  (pad G5 smd circle (at -3.2 -1.6) (size 0.35 0.35) (layers F.Cu F.Paste F.Mask) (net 7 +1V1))
  (pad F5 smd circle (at -3.2 -2.4) (size 0.35 0.35) (layers F.Cu F.Paste F.Mask))
  (pad E5 smd circle (at -3.2 -3.2) (size 0.35 0.35) (layers F.Cu F.Paste F.Mask) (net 6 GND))
  (pad D5 smd circle (at -3.2 -4) (size 0.35 0.35) (layers F.Cu F.Paste F.Mask))
  (pad C5 smd circle (at -3.2 -4.8) (size 0.35 0.35) (layers F.Cu F.Paste F.Mask))
  (pad B5 smd circle (at -3.2 -5.6) (size 0.35 0.35) (layers F.Cu F.Paste F.Mask))
  (pad A5 smd circle (at -3.2 -6.4) (size 0.35 0.35) (layers F.Cu F.Paste F.Mask))
  (pad U4 smd circle (at -4 6.4) (size 0.35 0.35) (layers F.Cu F.Paste F.Mask))
  (pad T4 smd circle (at -4 5.6) (size 0.35 0.35) (layers F.Cu F.Paste F.Mask))
  (pad R4 smd circle (at -4 4.8) (size 0.35 0.35) (layers F.Cu F.Paste F.Mask))
  (pad P4 smd circle (at -4 4) (size 0.35 0.35) (layers F.Cu F.Paste F.Mask) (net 6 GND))
  (pad N4 smd circle (at -4 3.2) (size 0.35 0.35) (layers F.Cu F.Paste F.Mask))
  (pad M4 smd circle (at -4 2.4) (size 0.35 0.35) (layers F.Cu F.Paste F.Mask))
  (pad L4 smd circle (at -4 1.6) (size 0.35 0.35) (layers F.Cu F.Paste F.Mask))
  (pad K4 smd circle (at -4 0.8) (size 0.35 0.35) (layers F.Cu F.Paste F.Mask))
  (pad J4 smd circle (at -4 0) (size 0.35 0.35) (layers F.Cu F.Paste F.Mask))
  (pad H4 smd circle (at -4 -0.8) (size 0.35 0.35) (layers F.Cu F.Paste F.Mask))
  (pad G4 smd circle (at -4 -1.6) (size 0.35 0.35) (layers F.Cu F.Paste F.Mask))
  (pad F4 smd circle (at -4 -2.4) (size 0.35 0.35) (layers F.Cu F.Paste F.Mask))
  (pad E4 smd circle (at -4 -3.2) (size 0.35 0.35) (layers F.Cu F.Paste F.Mask))
  (pad D4 smd circle (at -4 -4) (size 0.35 0.35) (layers F.Cu F.Paste F.Mask) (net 6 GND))
  (pad C4 smd circle (at -4 -4.8) (size 0.35 0.35) (layers F.Cu F.Paste F.Mask))
  (pad B4 smd circle (at -4 -5.6) (size 0.35 0.35) (layers F.Cu F.Paste F.Mask))
  (pad A4 smd circle (at -4 -6.4) (size 0.35 0.35) (layers F.Cu F.Paste F.Mask))
  (pad U3 smd circle (at -4.8 6.4) (size 0.35 0.35) (layers F.Cu F.Paste F.Mask))
  (pad T3 smd circle (at -4.8 5.6) (size 0.35 0.35) (layers F.Cu F.Paste F.Mask))
  (pad R3 smd circle (at -4.8 4.8) (size 0.35 0.35) (layers F.Cu F.Paste F.Mask) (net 6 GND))
  (pad P3 smd circle (at -4.8 4) (size 0.35 0.35) (layers F.Cu F.Paste F.Mask))
  (pad N3 smd circle (at -4.8 3.2) (size 0.35 0.35) (layers F.Cu F.Paste F.Mask))
  (pad M3 smd circle (at -4.8 2.4) (size 0.35 0.35) (layers F.Cu F.Paste F.Mask))
  (pad L3 smd circle (at -4.8 1.6) (size 0.35 0.35) (layers F.Cu F.Paste F.Mask))
  (pad K3 smd circle (at -4.8 0.8) (size 0.35 0.35) (layers F.Cu F.Paste F.Mask))
  (pad J3 smd circle (at -4.8 0) (size 0.35 0.35) (layers F.Cu F.Paste F.Mask) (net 6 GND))
  (pad H3 smd circle (at -4.8 -0.8) (size 0.35 0.35) (layers F.Cu F.Paste F.Mask))
  (pad G3 smd circle (at -4.8 -1.6) (size 0.35 0.35) (layers F.Cu F.Paste F.Mask))
  (pad F3 smd circle (at -4.8 -2.4) (size 0.35 0.35) (layers F.Cu F.Paste F.Mask) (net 6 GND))
  (pad E3 smd circle (at -4.8 -3.2) (size 0.35 0.35) (layers F.Cu F.Paste F.Mask))
  (pad D3 smd circle (at -4.8 -4) (size 0.35 0.35) (layers F.Cu F.Paste F.Mask))
  (pad C3 smd circle (at -4.8 -4.8) (size 0.35 0.35) (layers F.Cu F.Paste F.Mask) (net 6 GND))
  (pad B3 smd circle (at -4.8 -5.6) (size 0.35 0.35) (layers F.Cu F.Paste F.Mask))
  (pad A3 smd circle (at -4.8 -6.4) (size 0.35 0.35) (layers F.Cu F.Paste F.Mask))
  (pad U2 smd circle (at -5.6 6.4) (size 0.35 0.35) (layers F.Cu F.Paste F.Mask))
  (pad T2 smd circle (at -5.6 5.6) (size 0.35 0.35) (layers F.Cu F.Paste F.Mask) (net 6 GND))
  (pad R2 smd circle (at -5.6 4.8) (size 0.35 0.35) (layers F.Cu F.Paste F.Mask))
  (pad P2 smd circle (at -5.6 4) (size 0.35 0.35) (layers F.Cu F.Paste F.Mask))
  (pad N2 smd circle (at -5.6 3.2) (size 0.35 0.35) (layers F.Cu F.Paste F.Mask))
  (pad L2 smd circle (at -5.6 1.6) (size 0.35 0.35) (layers F.Cu F.Paste F.Mask))
  (pad K2 smd circle (at -5.6 0.8) (size 0.35 0.35) (layers F.Cu F.Paste F.Mask))
  (pad J2 smd circle (at -5.6 0) (size 0.35 0.35) (layers F.Cu F.Paste F.Mask))
  (pad H2 smd circle (at -5.6 -0.8) (size 0.35 0.35) (layers F.Cu F.Paste F.Mask))
  (pad G2 smd circle (at -5.6 -1.6) (size 0.35 0.35) (layers F.Cu F.Paste F.Mask))
  (pad E2 smd circle (at -5.6 -3.2) (size 0.35 0.35) (layers F.Cu F.Paste F.Mask))
  (pad D2 smd circle (at -5.6 -4) (size 0.35 0.35) (layers F.Cu F.Paste F.Mask))
  (pad C2 smd circle (at -5.6 -4.8) (size 0.35 0.35) (layers F.Cu F.Paste F.Mask) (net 7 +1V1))
  (pad B2 smd circle (at -5.6 -5.6) (size 0.35 0.35) (layers F.Cu F.Paste F.Mask) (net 6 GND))
  (pad A2 smd circle (at -5.6 -6.4) (size 0.35 0.35) (layers F.Cu F.Paste F.Mask))
  (pad U1 smd circle (at -6.4 6.4) (size 0.35 0.35) (layers F.Cu F.Paste F.Mask) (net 6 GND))
  (pad T1 smd circle (at -6.4 5.6) (size 0.35 0.35) (layers F.Cu F.Paste F.Mask))
  (pad R1 smd circle (at -6.4 4.8) (size 0.35 0.35) (layers F.Cu F.Paste F.Mask))
  (pad P1 smd circle (at -6.4 4) (size 0.35 0.35) (layers F.Cu F.Paste F.Mask) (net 1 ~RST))
  (pad N1 smd circle (at -6.4 3.2) (size 0.35 0.35) (layers F.Cu F.Paste F.Mask))
  (pad L1 smd circle (at -6.4 1.6) (size 0.35 0.35) (layers F.Cu F.Paste F.Mask))
  (pad K1 smd circle (at -6.4 0.8) (size 0.35 0.35) (layers F.Cu F.Paste F.Mask))
  (pad J1 smd circle (at -6.4 0) (size 0.35 0.35) (layers F.Cu F.Paste F.Mask))
  (pad H1 smd circle (at -6.4 -0.8) (size 0.35 0.35) (layers F.Cu F.Paste F.Mask))
  (pad G1 smd circle (at -6.4 -1.6) (size 0.35 0.35) (layers F.Cu F.Paste F.Mask))
  (pad E1 smd circle (at -6.4 -3.2) (size 0.35 0.35) (layers F.Cu F.Paste F.Mask))
  (pad D1 smd circle (at -6.4 -4) (size 0.35 0.35) (layers F.Cu F.Paste F.Mask))
  (pad C1 smd circle (at -6.4 -4.8) (size 0.35 0.35) (layers F.Cu F.Paste F.Mask))
  (pad B1 smd circle (at -6.4 -5.6) (size 0.35 0.35) (layers F.Cu F.Paste F.Mask))
  (pad A1 smd circle (at -6.4 -6.4) (size 0.35 0.35) (layers F.Cu F.Paste F.Mask) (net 6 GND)))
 (gr_line (start 225 60) (end 225 230) (layer Edge.Cuts) (width 0.1))
 (gr_line (start 55 60) (end 225 60) (layer Edge.Cuts) (width 0.1))
 (gr_line (start 55 230) (end 55 60) (layer Edge.Cuts) (width 0.1))
 (gr_line (start 225 230) (end 55 230) (layer Edge.Cuts) (width 0.1))
 (segment (start 211.7 139.65) (end 211.7 139.55) (width 0.15) (layer F.Cu) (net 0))
 (segment (start 144 141) (end 144.8 140.2) (width 0.15) (layer F.Cu) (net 6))
 (segment (start 139.2 144.2) (end 140.8 144.2) (width 0.15) (layer F.Cu) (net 6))
 (segment (start 140.8 144.2) (end 140.8 145.8) (width 0.15) (layer F.Cu) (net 6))
 (segment (start 140.8 145.8) (end 139.2 145.8) (width 0.15) (layer F.Cu) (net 6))
 (segment (start 139.2 145) (end 139.2 145.8) (width 0.15) (layer F.Cu) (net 6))
 (segment (start 139.2 145) (end 140.8 145) (width 0.15) (layer F.Cu) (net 6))
 (segment (start 139.2 145) (end 139.2 144.2) (width 0.15) (layer F.Cu) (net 6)))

